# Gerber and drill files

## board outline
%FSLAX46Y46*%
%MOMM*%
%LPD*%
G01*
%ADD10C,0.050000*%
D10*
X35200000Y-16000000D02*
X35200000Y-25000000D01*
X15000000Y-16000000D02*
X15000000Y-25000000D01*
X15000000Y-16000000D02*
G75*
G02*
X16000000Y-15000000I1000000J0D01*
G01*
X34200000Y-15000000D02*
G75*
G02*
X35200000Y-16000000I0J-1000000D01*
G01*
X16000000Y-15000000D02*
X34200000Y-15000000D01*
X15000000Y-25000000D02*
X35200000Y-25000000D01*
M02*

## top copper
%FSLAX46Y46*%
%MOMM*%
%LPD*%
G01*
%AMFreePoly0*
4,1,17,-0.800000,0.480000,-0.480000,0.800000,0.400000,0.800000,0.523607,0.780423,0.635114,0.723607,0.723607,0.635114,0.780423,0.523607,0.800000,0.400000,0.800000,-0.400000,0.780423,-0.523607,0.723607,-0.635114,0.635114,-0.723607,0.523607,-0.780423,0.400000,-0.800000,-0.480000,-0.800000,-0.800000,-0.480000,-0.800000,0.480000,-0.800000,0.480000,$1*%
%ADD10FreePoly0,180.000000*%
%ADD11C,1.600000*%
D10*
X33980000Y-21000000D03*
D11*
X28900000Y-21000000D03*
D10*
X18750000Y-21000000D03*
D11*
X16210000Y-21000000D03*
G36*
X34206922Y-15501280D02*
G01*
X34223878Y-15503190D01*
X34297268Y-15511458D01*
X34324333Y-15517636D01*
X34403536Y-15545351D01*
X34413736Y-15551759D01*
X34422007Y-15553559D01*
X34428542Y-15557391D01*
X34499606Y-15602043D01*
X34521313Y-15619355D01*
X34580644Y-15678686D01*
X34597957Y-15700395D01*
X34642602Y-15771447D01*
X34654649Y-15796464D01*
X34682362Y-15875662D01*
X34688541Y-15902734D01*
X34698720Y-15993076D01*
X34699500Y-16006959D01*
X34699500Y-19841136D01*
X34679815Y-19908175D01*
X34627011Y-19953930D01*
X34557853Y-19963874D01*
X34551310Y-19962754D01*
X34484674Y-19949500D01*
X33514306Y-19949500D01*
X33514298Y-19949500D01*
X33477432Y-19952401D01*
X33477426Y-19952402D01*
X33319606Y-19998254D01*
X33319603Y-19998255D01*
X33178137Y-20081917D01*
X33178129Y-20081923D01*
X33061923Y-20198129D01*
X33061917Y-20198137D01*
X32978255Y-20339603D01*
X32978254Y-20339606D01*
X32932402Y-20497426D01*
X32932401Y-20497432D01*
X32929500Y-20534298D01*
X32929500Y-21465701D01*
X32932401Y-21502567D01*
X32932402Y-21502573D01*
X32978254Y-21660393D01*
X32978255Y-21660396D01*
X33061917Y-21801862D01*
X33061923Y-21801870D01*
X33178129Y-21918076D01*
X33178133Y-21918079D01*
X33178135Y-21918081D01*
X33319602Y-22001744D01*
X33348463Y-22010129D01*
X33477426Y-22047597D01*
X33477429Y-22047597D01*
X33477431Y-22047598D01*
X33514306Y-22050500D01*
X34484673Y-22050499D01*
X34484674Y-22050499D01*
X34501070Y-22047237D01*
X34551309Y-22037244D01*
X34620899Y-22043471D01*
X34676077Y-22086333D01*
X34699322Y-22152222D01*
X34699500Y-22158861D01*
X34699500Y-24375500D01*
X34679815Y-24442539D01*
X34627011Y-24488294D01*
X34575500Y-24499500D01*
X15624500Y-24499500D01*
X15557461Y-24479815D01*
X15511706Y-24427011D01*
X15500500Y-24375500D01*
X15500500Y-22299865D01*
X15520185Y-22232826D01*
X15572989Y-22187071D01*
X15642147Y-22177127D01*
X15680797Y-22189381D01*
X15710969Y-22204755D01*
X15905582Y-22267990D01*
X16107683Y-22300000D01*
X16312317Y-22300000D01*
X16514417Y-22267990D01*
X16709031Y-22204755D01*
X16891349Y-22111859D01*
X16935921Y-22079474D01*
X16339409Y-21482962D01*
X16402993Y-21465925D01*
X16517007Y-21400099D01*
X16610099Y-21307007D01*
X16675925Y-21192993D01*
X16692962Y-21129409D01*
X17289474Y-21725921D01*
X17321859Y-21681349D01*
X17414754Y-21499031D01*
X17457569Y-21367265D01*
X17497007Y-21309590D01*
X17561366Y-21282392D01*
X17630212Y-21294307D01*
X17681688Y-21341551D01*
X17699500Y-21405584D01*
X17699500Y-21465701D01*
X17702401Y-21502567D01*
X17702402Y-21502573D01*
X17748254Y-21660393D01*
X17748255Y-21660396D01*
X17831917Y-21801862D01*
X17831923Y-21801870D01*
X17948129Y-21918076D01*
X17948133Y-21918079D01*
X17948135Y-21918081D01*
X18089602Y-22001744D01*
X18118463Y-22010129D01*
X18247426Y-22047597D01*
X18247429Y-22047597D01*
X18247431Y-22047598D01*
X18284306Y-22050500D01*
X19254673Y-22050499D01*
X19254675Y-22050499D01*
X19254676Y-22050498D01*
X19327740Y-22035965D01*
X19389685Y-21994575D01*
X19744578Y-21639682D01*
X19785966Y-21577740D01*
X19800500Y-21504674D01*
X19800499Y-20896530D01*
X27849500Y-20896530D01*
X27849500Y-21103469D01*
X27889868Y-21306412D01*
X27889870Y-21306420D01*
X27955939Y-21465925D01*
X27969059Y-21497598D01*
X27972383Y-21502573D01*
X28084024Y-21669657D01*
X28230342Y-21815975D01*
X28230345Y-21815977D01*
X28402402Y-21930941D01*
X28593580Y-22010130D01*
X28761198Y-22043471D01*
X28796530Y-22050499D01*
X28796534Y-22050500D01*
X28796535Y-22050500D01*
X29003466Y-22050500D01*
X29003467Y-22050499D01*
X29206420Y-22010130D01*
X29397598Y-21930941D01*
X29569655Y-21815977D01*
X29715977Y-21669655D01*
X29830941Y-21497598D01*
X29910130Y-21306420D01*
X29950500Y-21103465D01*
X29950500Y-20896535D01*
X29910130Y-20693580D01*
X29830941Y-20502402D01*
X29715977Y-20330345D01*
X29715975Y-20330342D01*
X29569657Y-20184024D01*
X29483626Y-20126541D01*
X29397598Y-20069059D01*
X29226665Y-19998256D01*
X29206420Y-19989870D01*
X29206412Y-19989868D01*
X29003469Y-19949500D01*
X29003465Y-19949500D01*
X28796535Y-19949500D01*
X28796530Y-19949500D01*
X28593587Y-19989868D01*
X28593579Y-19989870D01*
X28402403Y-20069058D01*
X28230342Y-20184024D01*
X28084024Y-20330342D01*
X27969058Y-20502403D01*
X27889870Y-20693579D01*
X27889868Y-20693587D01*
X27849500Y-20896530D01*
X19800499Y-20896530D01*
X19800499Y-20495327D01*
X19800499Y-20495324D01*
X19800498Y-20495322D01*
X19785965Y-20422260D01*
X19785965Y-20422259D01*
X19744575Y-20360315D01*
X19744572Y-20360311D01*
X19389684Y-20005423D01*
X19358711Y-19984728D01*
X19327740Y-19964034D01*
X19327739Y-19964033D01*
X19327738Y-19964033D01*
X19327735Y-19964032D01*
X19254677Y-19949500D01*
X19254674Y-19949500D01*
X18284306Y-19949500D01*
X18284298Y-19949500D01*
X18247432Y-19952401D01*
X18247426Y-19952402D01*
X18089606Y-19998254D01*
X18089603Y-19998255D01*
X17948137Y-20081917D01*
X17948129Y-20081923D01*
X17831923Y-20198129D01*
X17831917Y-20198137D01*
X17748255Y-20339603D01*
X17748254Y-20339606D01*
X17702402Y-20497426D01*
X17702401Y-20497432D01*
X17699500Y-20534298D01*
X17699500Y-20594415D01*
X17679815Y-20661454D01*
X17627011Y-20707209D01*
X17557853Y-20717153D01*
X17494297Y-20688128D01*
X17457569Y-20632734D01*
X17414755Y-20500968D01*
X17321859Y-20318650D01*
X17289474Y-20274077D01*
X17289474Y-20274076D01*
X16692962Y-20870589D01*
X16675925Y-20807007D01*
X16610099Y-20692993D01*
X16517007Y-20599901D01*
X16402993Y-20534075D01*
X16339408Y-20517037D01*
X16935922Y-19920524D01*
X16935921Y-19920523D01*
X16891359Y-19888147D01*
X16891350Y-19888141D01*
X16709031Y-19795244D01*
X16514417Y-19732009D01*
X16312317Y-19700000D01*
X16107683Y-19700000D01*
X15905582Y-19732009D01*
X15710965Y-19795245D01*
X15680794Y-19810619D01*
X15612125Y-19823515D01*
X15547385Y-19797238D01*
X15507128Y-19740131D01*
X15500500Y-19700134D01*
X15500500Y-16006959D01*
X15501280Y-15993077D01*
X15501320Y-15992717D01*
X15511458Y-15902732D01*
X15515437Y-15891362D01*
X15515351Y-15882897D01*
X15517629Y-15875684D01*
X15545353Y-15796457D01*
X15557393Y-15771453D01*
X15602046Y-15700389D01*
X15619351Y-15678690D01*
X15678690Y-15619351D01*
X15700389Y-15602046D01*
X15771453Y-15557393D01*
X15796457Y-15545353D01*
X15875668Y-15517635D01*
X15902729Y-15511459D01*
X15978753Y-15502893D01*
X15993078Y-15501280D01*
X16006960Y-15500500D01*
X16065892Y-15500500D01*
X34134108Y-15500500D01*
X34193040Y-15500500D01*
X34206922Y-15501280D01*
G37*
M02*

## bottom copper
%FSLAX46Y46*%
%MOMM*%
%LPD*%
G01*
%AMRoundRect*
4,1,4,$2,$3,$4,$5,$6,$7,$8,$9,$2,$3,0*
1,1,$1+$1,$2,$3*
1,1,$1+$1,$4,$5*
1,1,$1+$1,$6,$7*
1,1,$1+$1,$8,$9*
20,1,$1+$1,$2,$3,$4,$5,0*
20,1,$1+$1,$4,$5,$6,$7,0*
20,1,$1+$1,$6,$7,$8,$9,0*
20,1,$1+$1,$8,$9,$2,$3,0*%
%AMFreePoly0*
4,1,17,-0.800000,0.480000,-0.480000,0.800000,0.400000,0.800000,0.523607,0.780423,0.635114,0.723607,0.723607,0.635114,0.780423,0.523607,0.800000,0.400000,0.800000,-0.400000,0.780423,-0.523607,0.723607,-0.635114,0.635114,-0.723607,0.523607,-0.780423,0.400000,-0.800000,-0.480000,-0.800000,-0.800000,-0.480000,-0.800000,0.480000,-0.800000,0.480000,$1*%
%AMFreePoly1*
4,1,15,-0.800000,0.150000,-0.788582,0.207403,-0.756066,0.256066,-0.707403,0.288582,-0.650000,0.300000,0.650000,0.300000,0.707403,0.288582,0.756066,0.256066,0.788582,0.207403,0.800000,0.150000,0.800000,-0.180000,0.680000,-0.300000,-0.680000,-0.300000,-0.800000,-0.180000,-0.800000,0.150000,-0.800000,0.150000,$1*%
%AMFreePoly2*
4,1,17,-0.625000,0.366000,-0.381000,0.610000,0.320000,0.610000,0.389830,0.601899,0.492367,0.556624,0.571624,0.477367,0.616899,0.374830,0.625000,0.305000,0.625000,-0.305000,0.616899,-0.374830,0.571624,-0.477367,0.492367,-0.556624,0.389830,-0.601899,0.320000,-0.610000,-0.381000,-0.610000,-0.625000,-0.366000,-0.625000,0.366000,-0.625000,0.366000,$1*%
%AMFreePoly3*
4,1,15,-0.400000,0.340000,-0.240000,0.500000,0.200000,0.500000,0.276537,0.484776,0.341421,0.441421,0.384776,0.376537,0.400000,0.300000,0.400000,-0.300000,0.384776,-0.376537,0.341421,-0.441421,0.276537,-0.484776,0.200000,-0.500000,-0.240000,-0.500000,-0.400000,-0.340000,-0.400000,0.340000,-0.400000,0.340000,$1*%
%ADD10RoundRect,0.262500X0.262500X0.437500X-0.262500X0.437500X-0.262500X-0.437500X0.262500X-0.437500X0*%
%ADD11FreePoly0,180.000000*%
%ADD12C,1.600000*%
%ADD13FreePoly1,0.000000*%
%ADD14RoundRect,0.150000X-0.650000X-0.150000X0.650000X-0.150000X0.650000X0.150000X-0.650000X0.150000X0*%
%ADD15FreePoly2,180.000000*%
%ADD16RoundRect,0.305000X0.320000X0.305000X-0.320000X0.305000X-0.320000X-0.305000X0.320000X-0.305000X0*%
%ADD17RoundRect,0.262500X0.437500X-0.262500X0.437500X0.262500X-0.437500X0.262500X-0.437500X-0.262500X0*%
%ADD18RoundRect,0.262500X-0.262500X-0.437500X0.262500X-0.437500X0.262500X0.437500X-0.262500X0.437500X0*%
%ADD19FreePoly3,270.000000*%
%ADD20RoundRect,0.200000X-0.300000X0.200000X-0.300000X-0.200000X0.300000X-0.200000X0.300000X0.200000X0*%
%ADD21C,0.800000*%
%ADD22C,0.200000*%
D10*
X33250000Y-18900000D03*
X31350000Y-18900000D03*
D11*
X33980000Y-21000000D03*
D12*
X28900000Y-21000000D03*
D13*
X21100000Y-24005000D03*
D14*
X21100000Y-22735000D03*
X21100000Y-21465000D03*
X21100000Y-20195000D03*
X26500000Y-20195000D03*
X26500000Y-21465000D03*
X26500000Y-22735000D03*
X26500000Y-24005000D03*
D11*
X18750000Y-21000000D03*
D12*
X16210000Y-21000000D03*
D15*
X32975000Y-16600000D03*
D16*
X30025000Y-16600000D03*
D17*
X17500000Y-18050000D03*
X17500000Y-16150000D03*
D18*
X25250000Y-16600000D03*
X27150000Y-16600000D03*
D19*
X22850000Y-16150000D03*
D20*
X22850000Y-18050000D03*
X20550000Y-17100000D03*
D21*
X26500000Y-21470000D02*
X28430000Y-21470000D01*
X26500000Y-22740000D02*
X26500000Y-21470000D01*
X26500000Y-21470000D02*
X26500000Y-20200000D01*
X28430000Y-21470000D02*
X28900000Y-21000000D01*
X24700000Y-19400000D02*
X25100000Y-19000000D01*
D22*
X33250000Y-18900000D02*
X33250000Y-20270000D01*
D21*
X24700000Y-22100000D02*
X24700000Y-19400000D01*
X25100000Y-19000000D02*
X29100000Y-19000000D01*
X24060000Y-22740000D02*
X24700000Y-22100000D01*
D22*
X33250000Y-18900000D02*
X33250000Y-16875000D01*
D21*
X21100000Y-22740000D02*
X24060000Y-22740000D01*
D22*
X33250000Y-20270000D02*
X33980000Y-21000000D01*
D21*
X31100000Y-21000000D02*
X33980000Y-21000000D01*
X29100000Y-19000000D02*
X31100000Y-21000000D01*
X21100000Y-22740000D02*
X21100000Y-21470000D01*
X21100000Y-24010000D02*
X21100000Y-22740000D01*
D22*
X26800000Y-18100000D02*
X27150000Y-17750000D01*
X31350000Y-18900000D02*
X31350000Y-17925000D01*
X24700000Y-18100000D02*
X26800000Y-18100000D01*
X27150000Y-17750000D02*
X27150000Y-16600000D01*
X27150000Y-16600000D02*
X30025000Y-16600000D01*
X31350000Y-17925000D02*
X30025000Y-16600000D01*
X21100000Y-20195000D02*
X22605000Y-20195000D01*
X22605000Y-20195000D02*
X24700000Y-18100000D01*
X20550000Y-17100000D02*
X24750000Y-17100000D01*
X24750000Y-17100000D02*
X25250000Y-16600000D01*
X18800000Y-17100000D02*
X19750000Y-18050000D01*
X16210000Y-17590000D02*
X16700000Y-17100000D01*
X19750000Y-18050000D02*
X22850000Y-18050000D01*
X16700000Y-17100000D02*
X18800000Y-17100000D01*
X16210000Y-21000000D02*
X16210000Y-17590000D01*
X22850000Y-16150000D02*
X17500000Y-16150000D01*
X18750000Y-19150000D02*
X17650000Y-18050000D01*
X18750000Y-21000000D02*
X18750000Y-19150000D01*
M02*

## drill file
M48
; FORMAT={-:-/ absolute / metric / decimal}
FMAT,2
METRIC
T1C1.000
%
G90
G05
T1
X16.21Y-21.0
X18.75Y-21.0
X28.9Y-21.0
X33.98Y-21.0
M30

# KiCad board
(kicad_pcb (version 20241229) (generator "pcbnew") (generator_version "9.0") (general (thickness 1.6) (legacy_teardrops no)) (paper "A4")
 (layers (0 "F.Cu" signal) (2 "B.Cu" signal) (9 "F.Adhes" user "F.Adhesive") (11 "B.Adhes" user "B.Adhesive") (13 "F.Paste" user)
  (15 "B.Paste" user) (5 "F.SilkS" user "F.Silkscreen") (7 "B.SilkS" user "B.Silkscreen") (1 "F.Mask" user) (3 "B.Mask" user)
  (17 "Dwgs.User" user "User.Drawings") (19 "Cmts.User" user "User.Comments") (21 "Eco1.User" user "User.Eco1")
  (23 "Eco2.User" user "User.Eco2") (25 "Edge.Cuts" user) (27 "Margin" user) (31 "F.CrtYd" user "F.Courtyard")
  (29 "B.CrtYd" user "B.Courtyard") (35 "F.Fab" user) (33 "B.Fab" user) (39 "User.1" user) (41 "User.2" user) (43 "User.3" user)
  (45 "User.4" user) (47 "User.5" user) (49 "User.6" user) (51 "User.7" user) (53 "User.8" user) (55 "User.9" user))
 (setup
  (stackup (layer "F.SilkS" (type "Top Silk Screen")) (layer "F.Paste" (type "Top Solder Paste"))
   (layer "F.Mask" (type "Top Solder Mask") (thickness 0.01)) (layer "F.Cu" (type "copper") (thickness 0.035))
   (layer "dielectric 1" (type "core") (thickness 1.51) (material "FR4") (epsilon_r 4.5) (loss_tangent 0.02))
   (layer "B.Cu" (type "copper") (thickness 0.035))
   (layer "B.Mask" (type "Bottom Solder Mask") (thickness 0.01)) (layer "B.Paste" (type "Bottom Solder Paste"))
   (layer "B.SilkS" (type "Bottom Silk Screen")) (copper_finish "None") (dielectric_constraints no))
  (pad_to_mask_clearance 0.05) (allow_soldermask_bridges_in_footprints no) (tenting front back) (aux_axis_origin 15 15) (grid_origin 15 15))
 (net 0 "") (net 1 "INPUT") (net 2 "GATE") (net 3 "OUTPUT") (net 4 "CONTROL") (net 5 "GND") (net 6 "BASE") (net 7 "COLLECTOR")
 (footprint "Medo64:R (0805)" (layer "B.Cu") (at 32.3 18.9 180)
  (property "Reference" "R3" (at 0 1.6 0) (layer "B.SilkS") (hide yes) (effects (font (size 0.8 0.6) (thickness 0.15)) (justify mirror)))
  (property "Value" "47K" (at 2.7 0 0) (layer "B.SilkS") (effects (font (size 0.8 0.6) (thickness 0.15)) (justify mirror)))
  (pad "1" smd roundrect (at -0.95 0 180) (size 1.05 1.4) (layers "B.Cu" "B.Mask" "B.Paste") (roundrect_rratio 0.25) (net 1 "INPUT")
   (thermal_bridge_angle 45))
  (pad "2" smd roundrect (at 0.95 0 180) (size 1.05 1.4) (layers "B.Cu" "B.Mask" "B.Paste") (roundrect_rratio 0.25) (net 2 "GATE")
   (thermal_bridge_angle 45)))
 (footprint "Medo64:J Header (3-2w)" (layer "B.Cu") (at 31.44 21 180)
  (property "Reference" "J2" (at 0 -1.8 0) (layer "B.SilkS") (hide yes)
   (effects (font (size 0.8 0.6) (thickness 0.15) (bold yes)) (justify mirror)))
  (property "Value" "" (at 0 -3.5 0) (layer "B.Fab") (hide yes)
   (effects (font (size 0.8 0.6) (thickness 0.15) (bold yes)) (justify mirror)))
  (pad "1" thru_hole roundrect (at -2.54 0 180) (size 1.6 1.6) (drill 1) (layers "*.Cu" "*.Mask") (remove_unused_layers no)
   (roundrect_rratio 0.25) (chamfer_ratio 0.2) (chamfer top_left bottom_left) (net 1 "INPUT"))
  (pad "3" thru_hole circle (at 2.54 0 180) (size 1.6 1.6) (drill 1) (layers "*.Cu" "*.Mask") (remove_unused_layers no) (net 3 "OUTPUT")))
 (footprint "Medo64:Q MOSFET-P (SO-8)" (layer "B.Cu") (at 23.8 22.1)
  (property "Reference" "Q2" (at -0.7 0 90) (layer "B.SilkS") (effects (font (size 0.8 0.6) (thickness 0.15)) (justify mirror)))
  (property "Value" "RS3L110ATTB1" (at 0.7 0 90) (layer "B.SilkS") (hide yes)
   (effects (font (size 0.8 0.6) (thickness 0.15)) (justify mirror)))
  (pad "1" smd roundrect (at -2.7 1.905) (size 1.6 0.6) (layers "B.Cu" "B.Mask" "B.Paste") (roundrect_rratio 0.25) (chamfer_ratio 0.2)
   (chamfer bottom_left bottom_right) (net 1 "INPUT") (thermal_bridge_angle 45))
  (pad "2" smd roundrect (at -2.7 0.635) (size 1.6 0.6) (layers "B.Cu" "B.Mask" "B.Paste") (roundrect_rratio 0.25) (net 1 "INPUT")
   (thermal_bridge_angle 45))
  (pad "3" smd roundrect (at -2.7 -0.635) (size 1.6 0.6) (layers "B.Cu" "B.Mask" "B.Paste") (roundrect_rratio 0.25) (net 1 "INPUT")
   (thermal_bridge_angle 45))
  (pad "4" smd roundrect (at -2.7 -1.905) (size 1.6 0.6) (layers "B.Cu" "B.Mask" "B.Paste") (roundrect_rratio 0.25) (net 2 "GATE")
   (thermal_bridge_angle 45))
  (pad "5" smd roundrect (at 2.7 -1.905) (size 1.6 0.6) (layers "B.Cu" "B.Mask" "B.Paste") (roundrect_rratio 0.25) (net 3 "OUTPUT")
   (thermal_bridge_angle 45))
  (pad "6" smd roundrect (at 2.7 -0.635) (size 1.6 0.6) (layers "B.Cu" "B.Mask" "B.Paste") (roundrect_rratio 0.25) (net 3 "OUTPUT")
   (thermal_bridge_angle 45))
  (pad "7" smd roundrect (at 2.7 0.635) (size 1.6 0.6) (layers "B.Cu" "B.Mask" "B.Paste") (roundrect_rratio 0.25) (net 3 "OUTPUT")
   (thermal_bridge_angle 45))
  (pad "8" smd roundrect (at 2.7 1.905) (size 1.6 0.6) (layers "B.Cu" "B.Mask" "B.Paste") (roundrect_rratio 0.25) (thermal_bridge_angle 45)))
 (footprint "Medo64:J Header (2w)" (layer "B.Cu") (at 17.48 21 180)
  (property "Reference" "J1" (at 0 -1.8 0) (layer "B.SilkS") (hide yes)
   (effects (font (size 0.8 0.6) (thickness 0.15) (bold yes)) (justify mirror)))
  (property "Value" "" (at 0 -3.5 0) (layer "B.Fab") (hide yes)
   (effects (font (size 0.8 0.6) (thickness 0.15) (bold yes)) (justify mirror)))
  (pad "1" thru_hole roundrect (at -1.27 0 180) (size 1.6 1.6) (drill 1) (layers "*.Cu" "*.Mask") (remove_unused_layers no)
   (roundrect_rratio 0.25) (chamfer_ratio 0.2) (chamfer top_left bottom_left) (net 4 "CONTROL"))
  (pad "2" thru_hole circle (at 1.27 0 180) (size 1.6 1.6) (drill 1) (layers "*.Cu" "*.Mask") (remove_unused_layers no) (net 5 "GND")))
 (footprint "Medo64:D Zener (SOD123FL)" (layer "B.Cu") (at 31.5 16.6 180)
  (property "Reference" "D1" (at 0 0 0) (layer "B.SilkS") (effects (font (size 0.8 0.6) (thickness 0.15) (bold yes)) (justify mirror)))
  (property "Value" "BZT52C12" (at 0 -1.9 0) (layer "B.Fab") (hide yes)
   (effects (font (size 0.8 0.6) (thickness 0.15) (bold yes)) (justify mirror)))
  (pad "1" smd roundrect (at -1.475 0 180) (size 1.25 1.22) (layers "B.Cu" "B.Mask" "B.Paste") (roundrect_rratio 0.25) (chamfer_ratio 0.2)
   (chamfer top_left bottom_left) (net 1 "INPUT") (thermal_bridge_angle 45))
  (pad "2" smd roundrect (at 1.475 0 180) (size 1.25 1.22) (layers "B.Cu" "B.Mask" "B.Paste") (roundrect_rratio 0.25) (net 2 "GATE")
   (thermal_bridge_angle 45)))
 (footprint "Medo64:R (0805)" (layer "B.Cu") (at 17.5 17.1 90)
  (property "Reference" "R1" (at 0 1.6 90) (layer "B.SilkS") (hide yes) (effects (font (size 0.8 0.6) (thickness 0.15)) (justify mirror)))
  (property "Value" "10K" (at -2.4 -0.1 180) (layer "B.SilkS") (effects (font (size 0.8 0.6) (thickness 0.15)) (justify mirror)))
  (pad "1" smd roundrect (at -0.95 0 90) (size 1.05 1.4) (layers "B.Cu" "B.Mask" "B.Paste") (roundrect_rratio 0.25) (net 4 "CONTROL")
   (thermal_bridge_angle 45))
  (pad "2" smd roundrect (at 0.95 0 90) (size 1.05 1.4) (layers "B.Cu" "B.Mask" "B.Paste") (roundrect_rratio 0.25) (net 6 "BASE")
   (thermal_bridge_angle 45)))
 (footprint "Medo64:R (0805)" (layer "B.Cu") (at 26.2 16.6)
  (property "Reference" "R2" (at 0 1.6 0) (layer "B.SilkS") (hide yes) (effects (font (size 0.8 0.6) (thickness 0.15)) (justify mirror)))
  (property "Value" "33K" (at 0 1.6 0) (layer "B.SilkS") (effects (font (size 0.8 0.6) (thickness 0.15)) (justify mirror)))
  (pad "1" smd roundrect (at -0.95 0) (size 1.05 1.4) (layers "B.Cu" "B.Mask" "B.Paste") (roundrect_rratio 0.25) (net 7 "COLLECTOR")
   (thermal_bridge_angle 45))
  (pad "2" smd roundrect (at 0.95 0) (size 1.05 1.4) (layers "B.Cu" "B.Mask" "B.Paste") (roundrect_rratio 0.25) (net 2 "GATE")
   (thermal_bridge_angle 45)))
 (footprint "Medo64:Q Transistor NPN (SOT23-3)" (layer "B.Cu") (at 21.7 17.1 -90)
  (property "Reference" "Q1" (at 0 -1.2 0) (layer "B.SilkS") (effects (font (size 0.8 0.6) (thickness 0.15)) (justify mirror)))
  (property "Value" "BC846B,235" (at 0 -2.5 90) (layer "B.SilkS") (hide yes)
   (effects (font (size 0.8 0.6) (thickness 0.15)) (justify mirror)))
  (pad "1" smd roundrect (at -0.95 -1.15 270) (size 0.8 1) (layers "B.Cu" "B.Mask" "B.Paste") (roundrect_rratio 0.25) (chamfer_ratio 0.2)
   (chamfer top_left bottom_left) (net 6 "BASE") (thermal_bridge_angle 45))
  (pad "2" smd roundrect (at 0.95 -1.15 270) (size 0.8 1) (layers "B.Cu" "B.Mask" "B.Paste") (roundrect_rratio 0.25) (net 5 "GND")
   (thermal_bridge_angle 45))
  (pad "3" smd roundrect (at 0 1.15 270) (size 0.8 1) (layers "B.Cu" "B.Mask" "B.Paste") (roundrect_rratio 0.25) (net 7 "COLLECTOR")
   (thermal_bridge_angle 45)))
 (gr_line (start 35.2 16) (end 35.2 25) (stroke (width 0.05) (type solid)) (locked yes) (layer "Edge.Cuts"))
 (gr_line (start 15 16) (end 15 25) (stroke (width 0.05) (type solid)) (locked yes) (layer "Edge.Cuts"))
 (gr_arc (start 15 16) (mid 15.292893 15.292893) (end 16 15) (stroke (width 0.05) (type solid)) (locked yes) (layer "Edge.Cuts"))
 (gr_arc (start 34.2 15) (mid 34.907107 15.292893) (end 35.2 16) (stroke (width 0.05) (type solid)) (locked yes) (layer "Edge.Cuts"))
 (gr_line (start 16 15) (end 34.2 15) (stroke (width 0.05) (type solid)) (locked yes) (layer "Edge.Cuts"))
 (gr_line (start 15 25) (end 35.2 25) (stroke (width 0.05) (type solid)) (locked yes) (layer "Edge.Cuts"))
 (segment (start 26.5 21.47) (end 28.43 21.47) (width 0.8) (layer "B.Cu") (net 3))
 (segment (start 26.5 22.74) (end 26.5 21.47) (width 0.8) (layer "B.Cu") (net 3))
 (segment (start 26.5 21.47) (end 26.5 20.2) (width 0.8) (layer "B.Cu") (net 3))
 (segment (start 28.43 21.47) (end 28.9 21) (width 0.8) (layer "B.Cu") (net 3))
 (segment (start 24.7 19.4) (end 25.1 19) (width 0.8) (layer "B.Cu") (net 1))
 (segment (start 33.25 18.9) (end 33.25 20.27) (width 0.2) (layer "B.Cu") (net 1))
 (segment (start 24.7 22.1) (end 24.7 19.4) (width 0.8) (layer "B.Cu") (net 1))
 (segment (start 25.1 19) (end 29.1 19) (width 0.8) (layer "B.Cu") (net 1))
 (segment (start 24.06 22.74) (end 24.7 22.1) (width 0.8) (layer "B.Cu") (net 1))
 (segment (start 33.25 18.9) (end 33.25 16.875) (width 0.2) (layer "B.Cu") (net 1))
 (segment (start 21.1 22.74) (end 24.06 22.74) (width 0.8) (layer "B.Cu") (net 1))
 (segment (start 33.25 20.27) (end 33.98 21) (width 0.2) (layer "B.Cu") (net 1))
 (segment (start 31.1 21) (end 33.98 21) (width 0.8) (layer "B.Cu") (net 1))
 (segment (start 29.1 19) (end 31.1 21) (width 0.8) (layer "B.Cu") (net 1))
 (segment (start 21.1 22.74) (end 21.1 21.47) (width 0.8) (layer "B.Cu") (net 1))
 (segment (start 21.1 24.01) (end 21.1 22.74) (width 0.8) (layer "B.Cu") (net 1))
 (segment (start 26.8 18.1) (end 27.15 17.75) (width 0.2) (layer "B.Cu") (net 2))
 (segment (start 31.35 18.9) (end 31.35 17.925) (width 0.2) (layer "B.Cu") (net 2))
 (segment (start 24.7 18.1) (end 26.8 18.1) (width 0.2) (layer "B.Cu") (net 2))
 (segment (start 27.15 17.75) (end 27.15 16.6) (width 0.2) (layer "B.Cu") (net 2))
 (segment (start 27.15 16.6) (end 30.025 16.6) (width 0.2) (layer "B.Cu") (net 2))
 (segment (start 31.35 17.925) (end 30.025 16.6) (width 0.2) (layer "B.Cu") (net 2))
 (segment (start 21.1 20.195) (end 22.605 20.195) (width 0.2) (layer "B.Cu") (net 2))
 (segment (start 22.605 20.195) (end 24.7 18.1) (width 0.2) (layer "B.Cu") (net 2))
 (segment (start 20.55 17.1) (end 24.75 17.1) (width 0.2) (layer "B.Cu") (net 7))
 (segment (start 24.75 17.1) (end 25.25 16.6) (width 0.2) (layer "B.Cu") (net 7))
 (segment (start 18.8 17.1) (end 19.75 18.05) (width 0.2) (layer "B.Cu") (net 5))
 (segment (start 16.21 17.59) (end 16.7 17.1) (width 0.2) (layer "B.Cu") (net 5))
 (segment (start 19.75 18.05) (end 22.85 18.05) (width 0.2) (layer "B.Cu") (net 5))
 (segment (start 16.7 17.1) (end 18.8 17.1) (width 0.2) (layer "B.Cu") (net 5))
 (segment (start 16.21 21) (end 16.21 17.59) (width 0.2) (layer "B.Cu") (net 5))
 (segment (start 22.85 16.15) (end 17.5 16.15) (width 0.2) (layer "B.Cu") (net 6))
 (segment (start 18.75 19.15) (end 17.65 18.05) (width 0.2) (layer "B.Cu") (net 4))
 (segment (start 18.75 21) (end 18.75 19.15) (width 0.2) (layer "B.Cu") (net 4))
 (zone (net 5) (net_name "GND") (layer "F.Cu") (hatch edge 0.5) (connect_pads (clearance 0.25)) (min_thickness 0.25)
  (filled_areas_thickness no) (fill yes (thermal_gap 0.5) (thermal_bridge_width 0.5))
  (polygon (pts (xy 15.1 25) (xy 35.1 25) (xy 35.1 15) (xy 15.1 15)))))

